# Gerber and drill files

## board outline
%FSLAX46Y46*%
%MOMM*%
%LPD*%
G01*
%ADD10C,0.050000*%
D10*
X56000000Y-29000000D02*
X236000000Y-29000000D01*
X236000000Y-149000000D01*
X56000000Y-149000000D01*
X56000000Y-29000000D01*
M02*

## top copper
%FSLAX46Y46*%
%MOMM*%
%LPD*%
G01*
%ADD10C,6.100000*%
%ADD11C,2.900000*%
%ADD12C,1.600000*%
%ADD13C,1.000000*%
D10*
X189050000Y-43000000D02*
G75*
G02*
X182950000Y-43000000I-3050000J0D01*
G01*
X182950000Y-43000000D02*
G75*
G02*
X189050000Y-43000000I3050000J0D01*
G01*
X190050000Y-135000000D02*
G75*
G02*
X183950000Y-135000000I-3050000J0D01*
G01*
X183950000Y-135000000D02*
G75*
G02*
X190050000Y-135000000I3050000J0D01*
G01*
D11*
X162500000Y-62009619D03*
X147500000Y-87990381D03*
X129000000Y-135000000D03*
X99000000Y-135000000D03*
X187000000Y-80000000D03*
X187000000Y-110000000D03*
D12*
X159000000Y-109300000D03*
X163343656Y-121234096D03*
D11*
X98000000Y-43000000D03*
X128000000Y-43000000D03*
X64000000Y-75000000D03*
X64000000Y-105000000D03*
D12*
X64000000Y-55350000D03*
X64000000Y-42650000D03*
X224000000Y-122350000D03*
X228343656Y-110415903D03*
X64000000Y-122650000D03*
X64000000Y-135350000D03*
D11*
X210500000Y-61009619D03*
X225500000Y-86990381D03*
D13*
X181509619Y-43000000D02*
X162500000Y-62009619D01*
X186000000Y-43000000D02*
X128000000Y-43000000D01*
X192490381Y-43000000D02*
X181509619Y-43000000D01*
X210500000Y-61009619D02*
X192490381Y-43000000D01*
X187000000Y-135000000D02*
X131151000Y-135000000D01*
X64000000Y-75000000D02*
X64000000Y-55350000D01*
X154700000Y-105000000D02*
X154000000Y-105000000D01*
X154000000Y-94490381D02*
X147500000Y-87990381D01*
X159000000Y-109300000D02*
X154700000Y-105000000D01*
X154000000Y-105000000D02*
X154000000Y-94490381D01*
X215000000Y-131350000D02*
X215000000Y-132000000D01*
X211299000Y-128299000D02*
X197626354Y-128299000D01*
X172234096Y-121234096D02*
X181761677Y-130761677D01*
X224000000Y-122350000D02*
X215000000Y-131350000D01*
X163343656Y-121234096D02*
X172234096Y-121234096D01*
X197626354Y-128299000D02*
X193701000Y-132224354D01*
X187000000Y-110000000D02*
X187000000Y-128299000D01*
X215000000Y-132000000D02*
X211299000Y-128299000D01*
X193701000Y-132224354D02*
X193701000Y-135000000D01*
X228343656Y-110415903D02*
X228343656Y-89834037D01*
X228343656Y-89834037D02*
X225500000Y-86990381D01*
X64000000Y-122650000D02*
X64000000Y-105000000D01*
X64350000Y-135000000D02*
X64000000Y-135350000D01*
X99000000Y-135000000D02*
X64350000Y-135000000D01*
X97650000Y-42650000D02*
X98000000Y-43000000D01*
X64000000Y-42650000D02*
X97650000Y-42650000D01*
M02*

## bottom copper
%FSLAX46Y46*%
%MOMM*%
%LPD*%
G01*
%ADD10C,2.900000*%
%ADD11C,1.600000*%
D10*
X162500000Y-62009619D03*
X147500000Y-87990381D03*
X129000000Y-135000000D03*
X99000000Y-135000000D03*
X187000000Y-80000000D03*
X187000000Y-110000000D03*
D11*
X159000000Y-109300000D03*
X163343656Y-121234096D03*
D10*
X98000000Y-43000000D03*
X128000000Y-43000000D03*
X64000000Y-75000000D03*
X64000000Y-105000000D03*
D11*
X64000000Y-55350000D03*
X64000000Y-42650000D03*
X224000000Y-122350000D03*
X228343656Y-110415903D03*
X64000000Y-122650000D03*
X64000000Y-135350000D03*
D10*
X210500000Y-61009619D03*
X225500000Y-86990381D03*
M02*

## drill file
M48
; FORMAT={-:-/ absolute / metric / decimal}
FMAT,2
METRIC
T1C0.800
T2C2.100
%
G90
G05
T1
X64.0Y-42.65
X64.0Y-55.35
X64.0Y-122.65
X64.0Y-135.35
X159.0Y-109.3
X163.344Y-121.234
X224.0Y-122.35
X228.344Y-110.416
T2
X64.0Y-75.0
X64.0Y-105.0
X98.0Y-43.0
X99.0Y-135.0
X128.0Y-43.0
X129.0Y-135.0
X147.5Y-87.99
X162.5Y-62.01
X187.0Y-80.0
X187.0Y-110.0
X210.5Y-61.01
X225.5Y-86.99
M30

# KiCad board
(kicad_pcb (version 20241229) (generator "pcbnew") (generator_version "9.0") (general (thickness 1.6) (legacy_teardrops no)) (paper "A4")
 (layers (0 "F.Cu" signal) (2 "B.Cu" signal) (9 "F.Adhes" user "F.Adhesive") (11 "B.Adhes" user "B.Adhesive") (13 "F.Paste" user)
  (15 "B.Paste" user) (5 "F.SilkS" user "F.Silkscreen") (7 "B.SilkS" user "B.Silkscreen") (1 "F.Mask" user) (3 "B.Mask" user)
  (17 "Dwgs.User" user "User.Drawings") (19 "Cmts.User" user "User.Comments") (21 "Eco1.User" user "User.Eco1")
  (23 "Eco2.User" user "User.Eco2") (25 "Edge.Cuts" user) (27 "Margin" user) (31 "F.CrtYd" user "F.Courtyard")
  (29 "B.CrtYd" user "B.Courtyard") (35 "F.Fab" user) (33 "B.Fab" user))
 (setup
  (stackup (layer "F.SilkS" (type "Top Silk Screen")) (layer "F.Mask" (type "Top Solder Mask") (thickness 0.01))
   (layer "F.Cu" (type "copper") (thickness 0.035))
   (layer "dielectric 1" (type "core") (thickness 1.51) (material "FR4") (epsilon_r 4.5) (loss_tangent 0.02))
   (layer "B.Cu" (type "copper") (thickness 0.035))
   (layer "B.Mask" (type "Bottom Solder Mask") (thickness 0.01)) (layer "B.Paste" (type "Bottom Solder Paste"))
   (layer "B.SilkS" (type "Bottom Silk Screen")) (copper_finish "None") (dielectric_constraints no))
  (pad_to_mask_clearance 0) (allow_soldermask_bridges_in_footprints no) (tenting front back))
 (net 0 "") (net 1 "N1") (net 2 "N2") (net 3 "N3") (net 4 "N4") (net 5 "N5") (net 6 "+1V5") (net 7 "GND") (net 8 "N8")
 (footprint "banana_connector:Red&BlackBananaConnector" (layer "F.Cu") (at 155 75 -120)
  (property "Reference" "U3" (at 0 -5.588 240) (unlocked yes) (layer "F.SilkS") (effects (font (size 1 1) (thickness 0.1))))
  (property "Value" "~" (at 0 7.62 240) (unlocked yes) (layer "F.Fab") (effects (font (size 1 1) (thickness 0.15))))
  (pad "1" thru_hole circle (at -15 0 240) (size 2.9 2.9) (drill 2.1) (layers "*.Cu" "*.Mask") (remove_unused_layers no) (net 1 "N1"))
  (pad "2" thru_hole circle (at 15 0 240) (size 2.9 2.9) (drill 2.1) (layers "*.Cu" "*.Mask") (remove_unused_layers no) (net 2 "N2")))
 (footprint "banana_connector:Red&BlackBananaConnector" (layer "F.Cu") (at 114 135 180)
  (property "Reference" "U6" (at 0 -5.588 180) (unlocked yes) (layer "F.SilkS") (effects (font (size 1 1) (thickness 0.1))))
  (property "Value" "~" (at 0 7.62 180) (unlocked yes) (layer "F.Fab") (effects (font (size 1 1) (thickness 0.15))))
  (pad "1" thru_hole circle (at -15 0 180) (size 2.9 2.9) (drill 2.1) (layers "*.Cu" "*.Mask") (remove_unused_layers no) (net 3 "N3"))
  (pad "2" thru_hole circle (at 15 0 180) (size 2.9 2.9) (drill 2.1) (layers "*.Cu" "*.Mask") (remove_unused_layers no) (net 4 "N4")))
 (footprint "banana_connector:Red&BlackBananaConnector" (layer "F.Cu") (at 187 95 -90)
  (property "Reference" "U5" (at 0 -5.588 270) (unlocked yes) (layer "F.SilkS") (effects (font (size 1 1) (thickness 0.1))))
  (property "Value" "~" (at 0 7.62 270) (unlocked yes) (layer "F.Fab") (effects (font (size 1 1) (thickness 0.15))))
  (pad "1" thru_hole circle (at -15 0 270) (size 2.9 2.9) (drill 2.1) (layers "*.Cu" "*.Mask") (remove_unused_layers no) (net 1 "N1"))
  (pad "2" thru_hole circle (at 15 0 270) (size 2.9 2.9) (drill 2.1) (layers "*.Cu" "*.Mask") (remove_unused_layers no) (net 3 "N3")))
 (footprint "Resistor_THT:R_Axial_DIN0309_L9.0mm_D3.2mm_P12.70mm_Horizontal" (layer "F.Cu") (at 159 109.3 -70)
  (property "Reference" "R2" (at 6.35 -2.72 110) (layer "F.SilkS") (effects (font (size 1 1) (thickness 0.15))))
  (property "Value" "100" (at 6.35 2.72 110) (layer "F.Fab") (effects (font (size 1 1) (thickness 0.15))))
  (pad "1" thru_hole circle (at 0 0 290) (size 1.6 1.6) (drill 0.8) (layers "*.Cu" "*.Mask") (remove_unused_layers no) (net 2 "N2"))
  (pad "2" thru_hole circle (at 12.7 0 290) (size 1.6 1.6) (drill 0.8) (layers "*.Cu" "*.Mask") (remove_unused_layers no) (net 3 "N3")))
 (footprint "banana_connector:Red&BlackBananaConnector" (layer "F.Cu") (at 113 43)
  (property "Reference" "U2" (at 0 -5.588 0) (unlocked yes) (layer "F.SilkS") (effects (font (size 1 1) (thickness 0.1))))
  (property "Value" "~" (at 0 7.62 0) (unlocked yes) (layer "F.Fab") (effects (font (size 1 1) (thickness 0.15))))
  (pad "1" thru_hole circle (at -15 0) (size 2.9 2.9) (drill 2.1) (layers "*.Cu" "*.Mask") (remove_unused_layers no) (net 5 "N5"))
  (pad "2" thru_hole circle (at 15 0) (size 2.9 2.9) (drill 2.1) (layers "*.Cu" "*.Mask") (remove_unused_layers no) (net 1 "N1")))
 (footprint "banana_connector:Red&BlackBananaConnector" (layer "F.Cu") (at 64 90 -90)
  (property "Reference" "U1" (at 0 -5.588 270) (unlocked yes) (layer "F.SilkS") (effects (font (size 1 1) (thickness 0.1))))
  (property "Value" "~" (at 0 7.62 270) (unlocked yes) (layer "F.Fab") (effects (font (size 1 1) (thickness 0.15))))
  (pad "1" thru_hole circle (at -15 0 270) (size 2.9 2.9) (drill 2.1) (layers "*.Cu" "*.Mask") (remove_unused_layers no) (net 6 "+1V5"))
  (pad "2" thru_hole circle (at 15 0 270) (size 2.9 2.9) (drill 2.1) (layers "*.Cu" "*.Mask") (remove_unused_layers no) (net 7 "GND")))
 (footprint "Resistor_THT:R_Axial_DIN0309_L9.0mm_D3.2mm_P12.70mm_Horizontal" (layer "F.Cu") (at 64 55.35 90)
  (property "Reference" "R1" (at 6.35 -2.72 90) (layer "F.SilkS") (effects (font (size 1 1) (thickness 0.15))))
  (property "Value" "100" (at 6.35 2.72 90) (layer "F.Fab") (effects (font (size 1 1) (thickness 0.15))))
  (pad "1" thru_hole circle (at 0 0 90) (size 1.6 1.6) (drill 0.8) (layers "*.Cu" "*.Mask") (remove_unused_layers no) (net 6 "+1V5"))
  (pad "2" thru_hole circle (at 12.7 0 90) (size 1.6 1.6) (drill 0.8) (layers "*.Cu" "*.Mask") (remove_unused_layers no) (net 5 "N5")))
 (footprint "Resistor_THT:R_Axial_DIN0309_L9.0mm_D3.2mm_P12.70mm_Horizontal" (layer "F.Cu") (at 224 122.35 70)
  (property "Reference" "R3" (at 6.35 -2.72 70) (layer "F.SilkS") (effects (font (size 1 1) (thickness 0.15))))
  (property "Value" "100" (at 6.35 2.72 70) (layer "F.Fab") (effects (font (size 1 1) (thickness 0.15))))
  (pad "1" thru_hole circle (at 0 0 70) (size 1.6 1.6) (drill 0.8) (layers "*.Cu" "*.Mask") (remove_unused_layers no) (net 3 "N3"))
  (pad "2" thru_hole circle (at 12.700001 0 70) (size 1.6 1.6) (drill 0.8) (layers "*.Cu" "*.Mask") (remove_unused_layers no) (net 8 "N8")))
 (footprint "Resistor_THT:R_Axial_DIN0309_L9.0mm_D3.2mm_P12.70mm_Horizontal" (layer "F.Cu") (at 64 122.65 -90)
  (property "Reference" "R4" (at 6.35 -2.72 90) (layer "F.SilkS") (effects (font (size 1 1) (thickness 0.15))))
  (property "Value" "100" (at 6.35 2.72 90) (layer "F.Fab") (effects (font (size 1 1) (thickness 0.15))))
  (pad "1" thru_hole circle (at 0 0 270) (size 1.6 1.6) (drill 0.8) (layers "*.Cu" "*.Mask") (remove_unused_layers no) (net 7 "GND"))
  (pad "2" thru_hole circle (at 12.7 0 270) (size 1.6 1.6) (drill 0.8) (layers "*.Cu" "*.Mask") (remove_unused_layers no) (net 4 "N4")))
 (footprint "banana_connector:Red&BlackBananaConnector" (layer "F.Cu") (at 218 74 -60)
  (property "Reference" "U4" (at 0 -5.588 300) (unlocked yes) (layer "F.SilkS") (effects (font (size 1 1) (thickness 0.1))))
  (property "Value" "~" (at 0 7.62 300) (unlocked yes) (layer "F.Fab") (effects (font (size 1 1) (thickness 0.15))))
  (pad "1" thru_hole circle (at -15 0 300) (size 2.9 2.9) (drill 2.1) (layers "*.Cu" "*.Mask") (remove_unused_layers no) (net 1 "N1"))
  (pad "2" thru_hole circle (at 15 0 300) (size 2.9 2.9) (drill 2.1) (layers "*.Cu" "*.Mask") (remove_unused_layers no) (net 8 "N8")))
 (gr_circle (center 186 43) (end 192 43) (stroke (width 0.2) (type solid)) (fill yes) (layer "F.Cu") (net 1))
 (gr_circle (center 187 135) (end 193 135) (stroke (width 0.2) (type solid)) (fill yes) (layer "F.Cu") (net 1))
 (gr_rect (start 56 29) (end 236 149) (stroke (width 0.05) (type solid)) (fill no) (layer "Edge.Cuts"))
 (segment (start 181.509619 43) (end 162.5 62.009619) (width 1) (layer "F.Cu") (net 1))
 (segment (start 186 43) (end 128 43) (width 1) (layer "F.Cu") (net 1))
 (segment (start 192.490381 43) (end 181.509619 43) (width 1) (layer "F.Cu") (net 1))
 (segment (start 210.5 61.009619) (end 192.490381 43) (width 1) (layer "F.Cu") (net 1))
 (segment (start 187 135) (end 131.151 135) (width 1) (layer "F.Cu") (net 1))
 (segment (start 64 75) (end 64 55.35) (width 1) (layer "F.Cu") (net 6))
 (segment (start 154.7 105) (end 154 105) (width 1) (layer "F.Cu") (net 2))
 (segment (start 154 94.490381) (end 147.5 87.990381) (width 1) (layer "F.Cu") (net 2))
 (segment (start 159 109.3) (end 154.7 105) (width 1) (layer "F.Cu") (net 2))
 (segment (start 154 105) (end 154 94.490381) (width 1) (layer "F.Cu") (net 2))
 (segment (start 215 131.35) (end 215 132) (width 1) (layer "F.Cu") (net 3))
 (segment (start 211.299 128.299) (end 197.626354 128.299) (width 1) (layer "F.Cu") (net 3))
 (segment (start 172.234096 121.234096) (end 181.761677 130.761677) (width 1) (layer "F.Cu") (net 3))
 (segment (start 224 122.35) (end 215 131.35) (width 1) (layer "F.Cu") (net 3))
 (segment (start 163.343656 121.234096) (end 172.234096 121.234096) (width 1) (layer "F.Cu") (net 3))
 (segment (start 197.626354 128.299) (end 193.701 132.224354) (width 1) (layer "F.Cu") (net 3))
 (segment (start 187 110) (end 187 128.299) (width 1) (layer "F.Cu") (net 3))
 (segment (start 215 132) (end 211.299 128.299) (width 1) (layer "F.Cu") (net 3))
 (segment (start 193.701 132.224354) (end 193.701 135) (width 1) (layer "F.Cu") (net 3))
 (segment (start 228.343656 110.415903) (end 228.343656 89.834037) (width 1) (layer "F.Cu") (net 8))
 (segment (start 228.343656 89.834037) (end 225.5 86.990381) (width 1) (layer "F.Cu") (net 8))
 (segment (start 64 122.65) (end 64 105) (width 1) (layer "F.Cu") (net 7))
 (segment (start 64.35 135) (end 64 135.35) (width 1) (layer "F.Cu") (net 4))
 (segment (start 99 135) (end 64.35 135) (width 1) (layer "F.Cu") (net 4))
 (segment (start 97.65 42.65) (end 98 43) (width 1) (layer "F.Cu") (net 5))
 (segment (start 64 42.65) (end 97.65 42.65) (width 1) (layer "F.Cu") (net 5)))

